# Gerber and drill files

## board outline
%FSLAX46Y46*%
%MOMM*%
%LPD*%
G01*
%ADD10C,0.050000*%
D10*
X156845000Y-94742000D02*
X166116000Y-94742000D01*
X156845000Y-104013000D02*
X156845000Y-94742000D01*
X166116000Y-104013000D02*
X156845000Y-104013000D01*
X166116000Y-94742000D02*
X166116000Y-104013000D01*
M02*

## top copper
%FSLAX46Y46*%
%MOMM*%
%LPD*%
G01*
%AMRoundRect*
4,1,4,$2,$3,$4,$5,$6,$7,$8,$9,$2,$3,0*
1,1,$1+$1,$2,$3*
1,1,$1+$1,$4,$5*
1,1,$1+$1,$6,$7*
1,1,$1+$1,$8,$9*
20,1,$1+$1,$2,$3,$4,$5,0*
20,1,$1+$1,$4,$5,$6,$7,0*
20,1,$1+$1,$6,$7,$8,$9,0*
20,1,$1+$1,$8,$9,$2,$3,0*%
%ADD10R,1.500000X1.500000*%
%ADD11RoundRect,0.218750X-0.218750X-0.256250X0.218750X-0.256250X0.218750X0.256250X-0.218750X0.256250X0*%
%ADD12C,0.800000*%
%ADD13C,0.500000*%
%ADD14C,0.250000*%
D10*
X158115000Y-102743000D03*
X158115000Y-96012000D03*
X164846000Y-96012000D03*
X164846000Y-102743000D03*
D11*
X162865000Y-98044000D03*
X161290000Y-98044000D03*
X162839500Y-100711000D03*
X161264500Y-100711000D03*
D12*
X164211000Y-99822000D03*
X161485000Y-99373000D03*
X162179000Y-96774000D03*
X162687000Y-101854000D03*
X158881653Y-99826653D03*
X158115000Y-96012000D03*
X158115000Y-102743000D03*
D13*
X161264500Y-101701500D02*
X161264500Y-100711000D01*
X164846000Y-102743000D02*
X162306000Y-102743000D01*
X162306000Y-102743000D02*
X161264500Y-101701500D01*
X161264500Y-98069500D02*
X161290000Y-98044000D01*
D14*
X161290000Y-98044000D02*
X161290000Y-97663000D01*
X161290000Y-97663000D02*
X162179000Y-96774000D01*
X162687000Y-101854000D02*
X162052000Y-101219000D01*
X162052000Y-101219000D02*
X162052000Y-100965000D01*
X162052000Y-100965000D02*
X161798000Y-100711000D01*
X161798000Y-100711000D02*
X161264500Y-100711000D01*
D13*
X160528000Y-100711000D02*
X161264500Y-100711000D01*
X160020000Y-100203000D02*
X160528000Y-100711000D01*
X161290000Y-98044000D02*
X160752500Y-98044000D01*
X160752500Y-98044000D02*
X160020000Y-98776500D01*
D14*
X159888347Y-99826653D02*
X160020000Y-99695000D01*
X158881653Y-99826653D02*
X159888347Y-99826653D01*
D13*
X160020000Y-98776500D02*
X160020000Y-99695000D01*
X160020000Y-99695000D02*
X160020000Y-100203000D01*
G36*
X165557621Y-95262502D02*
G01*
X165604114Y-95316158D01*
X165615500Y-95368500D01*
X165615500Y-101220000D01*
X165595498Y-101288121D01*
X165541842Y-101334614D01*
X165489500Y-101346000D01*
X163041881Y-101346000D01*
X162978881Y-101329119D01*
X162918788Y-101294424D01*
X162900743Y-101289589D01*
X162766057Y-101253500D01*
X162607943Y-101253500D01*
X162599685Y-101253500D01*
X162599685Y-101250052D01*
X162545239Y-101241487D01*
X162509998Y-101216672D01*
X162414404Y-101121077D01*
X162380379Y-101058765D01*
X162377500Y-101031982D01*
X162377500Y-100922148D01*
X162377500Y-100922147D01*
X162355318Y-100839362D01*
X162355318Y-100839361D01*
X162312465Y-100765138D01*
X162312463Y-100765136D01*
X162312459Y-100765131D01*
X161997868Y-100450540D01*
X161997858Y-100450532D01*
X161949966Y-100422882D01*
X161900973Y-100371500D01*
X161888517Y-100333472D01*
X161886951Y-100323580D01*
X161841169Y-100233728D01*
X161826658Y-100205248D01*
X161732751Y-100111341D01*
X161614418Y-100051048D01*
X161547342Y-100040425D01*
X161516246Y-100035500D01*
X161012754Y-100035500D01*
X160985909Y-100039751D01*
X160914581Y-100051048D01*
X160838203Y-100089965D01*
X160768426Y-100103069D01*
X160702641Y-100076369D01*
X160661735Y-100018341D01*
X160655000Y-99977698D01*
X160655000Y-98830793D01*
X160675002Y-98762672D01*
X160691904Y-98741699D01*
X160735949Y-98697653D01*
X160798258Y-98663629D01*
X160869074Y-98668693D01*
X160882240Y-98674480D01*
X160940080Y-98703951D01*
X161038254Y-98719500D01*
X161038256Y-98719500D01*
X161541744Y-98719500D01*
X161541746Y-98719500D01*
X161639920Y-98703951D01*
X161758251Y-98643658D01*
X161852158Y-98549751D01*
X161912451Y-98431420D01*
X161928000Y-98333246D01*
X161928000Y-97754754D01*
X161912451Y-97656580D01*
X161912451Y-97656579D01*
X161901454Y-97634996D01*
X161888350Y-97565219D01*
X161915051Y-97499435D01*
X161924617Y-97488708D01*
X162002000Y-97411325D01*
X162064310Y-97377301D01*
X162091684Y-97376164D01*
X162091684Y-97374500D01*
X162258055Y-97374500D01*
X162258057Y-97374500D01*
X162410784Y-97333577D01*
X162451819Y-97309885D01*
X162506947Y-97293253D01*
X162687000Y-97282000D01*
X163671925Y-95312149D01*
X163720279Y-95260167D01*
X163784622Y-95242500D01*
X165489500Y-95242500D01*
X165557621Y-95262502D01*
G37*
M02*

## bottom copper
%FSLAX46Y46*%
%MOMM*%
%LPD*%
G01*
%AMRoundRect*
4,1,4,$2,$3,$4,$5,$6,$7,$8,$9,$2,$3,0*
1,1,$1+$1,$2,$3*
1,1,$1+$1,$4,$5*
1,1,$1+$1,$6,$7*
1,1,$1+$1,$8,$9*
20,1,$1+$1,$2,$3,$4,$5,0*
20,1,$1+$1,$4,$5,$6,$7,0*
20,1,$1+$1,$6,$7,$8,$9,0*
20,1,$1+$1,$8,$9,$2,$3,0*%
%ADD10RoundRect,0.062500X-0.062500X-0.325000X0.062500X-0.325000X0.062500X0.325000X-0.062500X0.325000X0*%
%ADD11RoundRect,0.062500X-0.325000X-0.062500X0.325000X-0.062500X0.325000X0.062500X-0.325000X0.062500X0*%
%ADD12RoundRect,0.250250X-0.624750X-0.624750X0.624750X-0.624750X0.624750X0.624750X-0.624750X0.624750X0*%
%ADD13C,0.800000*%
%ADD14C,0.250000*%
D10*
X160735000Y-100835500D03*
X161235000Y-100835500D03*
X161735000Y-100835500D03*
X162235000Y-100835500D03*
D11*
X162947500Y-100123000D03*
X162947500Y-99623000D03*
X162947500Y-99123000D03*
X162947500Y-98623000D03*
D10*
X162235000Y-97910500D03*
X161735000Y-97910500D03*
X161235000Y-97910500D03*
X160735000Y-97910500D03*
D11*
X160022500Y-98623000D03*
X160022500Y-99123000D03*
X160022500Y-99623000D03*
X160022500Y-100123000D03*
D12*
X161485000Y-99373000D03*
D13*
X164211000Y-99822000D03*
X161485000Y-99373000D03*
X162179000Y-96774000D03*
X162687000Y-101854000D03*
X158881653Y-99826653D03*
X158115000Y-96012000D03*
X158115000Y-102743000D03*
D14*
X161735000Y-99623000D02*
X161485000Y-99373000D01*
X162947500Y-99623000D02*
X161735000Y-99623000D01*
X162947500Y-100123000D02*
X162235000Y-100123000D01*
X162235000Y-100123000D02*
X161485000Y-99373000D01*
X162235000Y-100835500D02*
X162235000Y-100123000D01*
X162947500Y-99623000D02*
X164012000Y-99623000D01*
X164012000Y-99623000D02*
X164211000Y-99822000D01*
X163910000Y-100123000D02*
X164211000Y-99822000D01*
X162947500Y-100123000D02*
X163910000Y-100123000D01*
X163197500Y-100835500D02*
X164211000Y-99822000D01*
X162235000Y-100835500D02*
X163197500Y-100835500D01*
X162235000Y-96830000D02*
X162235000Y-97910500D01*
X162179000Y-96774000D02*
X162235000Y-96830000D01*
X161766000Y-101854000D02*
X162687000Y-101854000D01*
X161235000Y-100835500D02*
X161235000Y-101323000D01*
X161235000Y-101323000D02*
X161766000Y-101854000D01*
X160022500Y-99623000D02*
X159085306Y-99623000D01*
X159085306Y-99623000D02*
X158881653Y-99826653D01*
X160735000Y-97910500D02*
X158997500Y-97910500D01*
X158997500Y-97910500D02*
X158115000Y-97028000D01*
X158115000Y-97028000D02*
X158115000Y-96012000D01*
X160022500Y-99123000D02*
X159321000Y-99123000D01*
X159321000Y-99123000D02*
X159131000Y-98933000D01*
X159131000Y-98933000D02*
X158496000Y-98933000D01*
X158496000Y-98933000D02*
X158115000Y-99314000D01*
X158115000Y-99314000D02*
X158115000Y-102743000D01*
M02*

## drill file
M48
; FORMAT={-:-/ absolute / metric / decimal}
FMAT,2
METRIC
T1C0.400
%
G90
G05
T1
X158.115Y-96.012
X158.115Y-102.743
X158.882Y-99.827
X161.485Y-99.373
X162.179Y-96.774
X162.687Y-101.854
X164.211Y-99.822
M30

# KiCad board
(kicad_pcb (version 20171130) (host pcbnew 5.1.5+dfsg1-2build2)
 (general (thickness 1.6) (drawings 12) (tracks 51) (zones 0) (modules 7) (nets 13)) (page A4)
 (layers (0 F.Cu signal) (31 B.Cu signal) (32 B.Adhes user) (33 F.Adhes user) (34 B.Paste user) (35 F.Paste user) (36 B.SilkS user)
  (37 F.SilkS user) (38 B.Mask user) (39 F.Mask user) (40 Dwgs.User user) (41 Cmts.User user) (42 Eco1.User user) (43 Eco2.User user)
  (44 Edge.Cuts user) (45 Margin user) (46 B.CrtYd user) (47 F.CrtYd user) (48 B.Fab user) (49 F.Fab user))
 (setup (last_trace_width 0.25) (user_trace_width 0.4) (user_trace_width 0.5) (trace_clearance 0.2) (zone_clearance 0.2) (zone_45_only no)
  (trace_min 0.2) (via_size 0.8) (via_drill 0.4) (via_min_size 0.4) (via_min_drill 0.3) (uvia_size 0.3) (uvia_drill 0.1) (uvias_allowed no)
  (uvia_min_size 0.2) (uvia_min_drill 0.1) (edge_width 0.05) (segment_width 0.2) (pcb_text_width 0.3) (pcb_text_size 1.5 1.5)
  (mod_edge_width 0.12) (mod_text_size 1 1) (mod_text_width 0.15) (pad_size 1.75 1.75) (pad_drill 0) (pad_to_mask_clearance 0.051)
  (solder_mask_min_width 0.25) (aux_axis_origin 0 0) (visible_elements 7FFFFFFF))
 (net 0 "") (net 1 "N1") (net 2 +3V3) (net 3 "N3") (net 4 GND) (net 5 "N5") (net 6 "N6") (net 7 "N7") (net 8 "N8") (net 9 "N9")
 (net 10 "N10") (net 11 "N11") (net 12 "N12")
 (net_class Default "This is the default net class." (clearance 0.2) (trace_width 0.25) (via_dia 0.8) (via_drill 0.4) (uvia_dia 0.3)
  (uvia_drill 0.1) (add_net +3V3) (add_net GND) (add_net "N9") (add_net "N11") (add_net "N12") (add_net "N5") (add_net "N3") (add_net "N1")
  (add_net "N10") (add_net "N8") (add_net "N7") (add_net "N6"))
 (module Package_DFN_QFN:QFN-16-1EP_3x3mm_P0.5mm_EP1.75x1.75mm (layer B.Cu) (at 161.485 99.373)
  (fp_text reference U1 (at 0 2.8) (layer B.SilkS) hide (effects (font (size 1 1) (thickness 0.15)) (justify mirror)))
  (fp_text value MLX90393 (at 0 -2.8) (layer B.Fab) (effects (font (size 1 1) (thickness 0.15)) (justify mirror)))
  (pad 16 smd roundrect (at -0.75 1.4625) (size 0.25 0.775) (layers B.Cu B.Paste B.Mask) (roundrect_rratio 0.25) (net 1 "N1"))
  (pad 15 smd roundrect (at -0.25 1.4625) (size 0.25 0.775) (layers B.Cu B.Paste B.Mask) (roundrect_rratio 0.25) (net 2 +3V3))
  (pad 14 smd roundrect (at 0.25 1.4625) (size 0.25 0.775) (layers B.Cu B.Paste B.Mask) (roundrect_rratio 0.25) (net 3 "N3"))
  (pad 13 smd roundrect (at 0.75 1.4625) (size 0.25 0.775) (layers B.Cu B.Paste B.Mask) (roundrect_rratio 0.25) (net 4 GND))
  (pad 12 smd roundrect (at 1.4625 0.75) (size 0.775 0.25) (layers B.Cu B.Paste B.Mask) (roundrect_rratio 0.25) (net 4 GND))
  (pad 11 smd roundrect (at 1.4625 0.25) (size 0.775 0.25) (layers B.Cu B.Paste B.Mask) (roundrect_rratio 0.25) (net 4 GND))
  (pad 10 smd roundrect (at 1.4625 -0.25) (size 0.775 0.25) (layers B.Cu B.Paste B.Mask) (roundrect_rratio 0.25) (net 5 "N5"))
  (pad 9 smd roundrect (at 1.4625 -0.75) (size 0.775 0.25) (layers B.Cu B.Paste B.Mask) (roundrect_rratio 0.25) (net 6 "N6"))
  (pad 8 smd roundrect (at 0.75 -1.4625) (size 0.25 0.775) (layers B.Cu B.Paste B.Mask) (roundrect_rratio 0.25) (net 2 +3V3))
  (pad 7 smd roundrect (at 0.25 -1.4625) (size 0.25 0.775) (layers B.Cu B.Paste B.Mask) (roundrect_rratio 0.25) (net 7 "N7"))
  (pad 6 smd roundrect (at -0.25 -1.4625) (size 0.25 0.775) (layers B.Cu B.Paste B.Mask) (roundrect_rratio 0.25) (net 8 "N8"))
  (pad 5 smd roundrect (at -0.75 -1.4625) (size 0.25 0.775) (layers B.Cu B.Paste B.Mask) (roundrect_rratio 0.25) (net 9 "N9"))
  (pad 4 smd roundrect (at -1.4625 -0.75) (size 0.775 0.25) (layers B.Cu B.Paste B.Mask) (roundrect_rratio 0.25) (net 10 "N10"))
  (pad 3 smd roundrect (at -1.4625 -0.25) (size 0.775 0.25) (layers B.Cu B.Paste B.Mask) (roundrect_rratio 0.25) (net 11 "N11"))
  (pad 2 smd roundrect (at -1.4625 0.25) (size 0.775 0.25) (layers B.Cu B.Paste B.Mask) (roundrect_rratio 0.25) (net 2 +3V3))
  (pad 1 smd roundrect (at -1.4625 0.75) (size 0.775 0.25) (layers B.Cu B.Paste B.Mask) (roundrect_rratio 0.25) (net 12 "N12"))
  (pad "" smd roundrect (at 0.44 -0.44) (size 0.71 0.71) (layers B.Paste) (roundrect_rratio 0.25))
  (pad "" smd roundrect (at 0.44 0.44) (size 0.71 0.71) (layers B.Paste) (roundrect_rratio 0.25))
  (pad "" smd roundrect (at -0.44 -0.44) (size 0.71 0.71) (layers B.Paste) (roundrect_rratio 0.25))
  (pad "" smd roundrect (at -0.44 0.44) (size 0.71 0.71) (layers B.Paste) (roundrect_rratio 0.25))
  (pad 17 smd roundrect (at 0 0) (size 1.75 1.75) (layers B.Cu B.Mask) (roundrect_rratio 0.143) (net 4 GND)))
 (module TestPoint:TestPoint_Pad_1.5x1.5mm (layer F.Cu) (at 158.115 102.743)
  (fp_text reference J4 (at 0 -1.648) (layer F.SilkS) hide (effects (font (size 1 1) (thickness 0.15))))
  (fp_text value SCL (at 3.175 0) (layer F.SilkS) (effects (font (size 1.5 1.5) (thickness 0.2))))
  (pad 1 smd rect (at 0 0) (size 1.5 1.5) (layers F.Cu F.Mask) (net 11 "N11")))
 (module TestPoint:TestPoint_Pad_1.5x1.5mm (layer F.Cu) (at 158.115 96.012)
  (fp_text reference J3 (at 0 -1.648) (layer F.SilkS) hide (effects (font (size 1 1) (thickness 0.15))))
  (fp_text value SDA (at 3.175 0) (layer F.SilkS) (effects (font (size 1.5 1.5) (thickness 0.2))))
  (pad 1 smd rect (at 0 0) (size 1.5 1.5) (layers F.Cu F.Mask) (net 9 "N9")))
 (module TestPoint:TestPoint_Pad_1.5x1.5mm (layer F.Cu) (at 164.846 96.012)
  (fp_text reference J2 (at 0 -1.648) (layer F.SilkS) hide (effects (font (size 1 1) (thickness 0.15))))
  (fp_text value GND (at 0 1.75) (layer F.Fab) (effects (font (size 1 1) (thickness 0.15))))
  (pad 1 smd rect (at 0 0) (size 1.5 1.5) (layers F.Cu F.Mask) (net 4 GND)))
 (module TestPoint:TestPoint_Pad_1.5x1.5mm (layer F.Cu) (at 164.846 102.743)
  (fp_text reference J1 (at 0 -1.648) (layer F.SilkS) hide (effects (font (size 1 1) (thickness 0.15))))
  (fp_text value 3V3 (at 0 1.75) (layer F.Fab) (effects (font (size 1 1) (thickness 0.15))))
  (pad 1 smd rect (at 0 0) (size 1.5 1.5) (layers F.Cu F.Mask) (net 2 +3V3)))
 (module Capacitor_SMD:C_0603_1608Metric (layer F.Cu) (at 162.0775 98.044)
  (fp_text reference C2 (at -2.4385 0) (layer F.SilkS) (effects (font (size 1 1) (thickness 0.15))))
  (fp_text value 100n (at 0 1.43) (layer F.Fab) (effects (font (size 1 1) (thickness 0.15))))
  (pad 2 smd roundrect (at 0.7875 0) (size 0.875 0.95) (layers F.Cu F.Paste F.Mask) (roundrect_rratio 0.25) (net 4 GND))
  (pad 1 smd roundrect (at -0.7875 0) (size 0.875 0.95) (layers F.Cu F.Paste F.Mask) (roundrect_rratio 0.25) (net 2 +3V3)))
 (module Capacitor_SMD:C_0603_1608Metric (layer F.Cu) (at 162.052 100.711)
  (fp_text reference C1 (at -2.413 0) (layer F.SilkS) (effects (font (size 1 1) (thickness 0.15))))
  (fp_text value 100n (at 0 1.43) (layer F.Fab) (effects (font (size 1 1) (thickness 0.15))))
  (pad 2 smd roundrect (at 0.7875 0) (size 0.875 0.95) (layers F.Cu F.Paste F.Mask) (roundrect_rratio 0.25) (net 4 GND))
  (pad 1 smd roundrect (at -0.7875 0) (size 0.875 0.95) (layers F.Cu F.Paste F.Mask) (roundrect_rratio 0.25) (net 2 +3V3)))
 (gr_line (start 156.845 94.742) (end 166.116 94.742) (layer Edge.Cuts) (width 0.05))
 (gr_line (start 156.845 104.013) (end 156.845 94.742) (layer Edge.Cuts) (width 0.05))
 (gr_line (start 166.116 104.013) (end 156.845 104.013) (layer Edge.Cuts) (width 0.05))
 (gr_line (start 166.116 94.742) (end 166.116 104.013) (layer Edge.Cuts) (width 0.05))
 (segment (start 161.735 99.623) (end 161.485 99.373) (width 0.25) (layer B.Cu) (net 4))
 (segment (start 162.9475 99.623) (end 161.735 99.623) (width 0.25) (layer B.Cu) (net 4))
 (segment (start 162.9475 100.123) (end 162.235 100.123) (width 0.25) (layer B.Cu) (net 4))
 (segment (start 162.235 100.123) (end 161.485 99.373) (width 0.25) (layer B.Cu) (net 4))
 (segment (start 162.235 100.8355) (end 162.235 100.123) (width 0.25) (layer B.Cu) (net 4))
 (via (at 164.211 99.822) (size 0.8) (drill 0.4) (layers F.Cu B.Cu) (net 4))
 (segment (start 162.9475 99.623) (end 164.012 99.623) (width 0.25) (layer B.Cu) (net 4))
 (segment (start 164.012 99.623) (end 164.211 99.822) (width 0.25) (layer B.Cu) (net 4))
 (segment (start 163.91 100.123) (end 164.211 99.822) (width 0.25) (layer B.Cu) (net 4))
 (segment (start 162.9475 100.123) (end 163.91 100.123) (width 0.25) (layer B.Cu) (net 4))
 (segment (start 163.1975 100.8355) (end 164.211 99.822) (width 0.25) (layer B.Cu) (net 4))
 (segment (start 162.235 100.8355) (end 163.1975 100.8355) (width 0.25) (layer B.Cu) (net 4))
 (via (at 161.485 99.373) (size 0.8) (drill 0.4) (layers F.Cu B.Cu) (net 4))
 (segment (start 161.2645 101.7015) (end 161.2645 100.711) (width 0.5) (layer F.Cu) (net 2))
 (segment (start 164.846 102.743) (end 162.306 102.743) (width 0.5) (layer F.Cu) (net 2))
 (segment (start 162.306 102.743) (end 161.2645 101.7015) (width 0.5) (layer F.Cu) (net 2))
 (segment (start 161.2645 98.0695) (end 161.29 98.044) (width 0.5) (layer F.Cu) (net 2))
 (via (at 162.179 96.774) (size 0.8) (drill 0.4) (layers F.Cu B.Cu) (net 2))
 (segment (start 161.29 98.044) (end 161.29 97.663) (width 0.25) (layer F.Cu) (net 2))
 (segment (start 161.29 97.663) (end 162.179 96.774) (width 0.25) (layer F.Cu) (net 2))
 (segment (start 162.235 96.83) (end 162.235 97.9105) (width 0.25) (layer B.Cu) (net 2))
 (segment (start 162.179 96.774) (end 162.235 96.83) (width 0.25) (layer B.Cu) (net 2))
 (via (at 162.687 101.854) (size 0.8) (drill 0.4) (layers F.Cu B.Cu) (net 2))
 (segment (start 161.766 101.854) (end 162.687 101.854) (width 0.25) (layer B.Cu) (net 2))
 (segment (start 161.235 100.8355) (end 161.235 101.323) (width 0.25) (layer B.Cu) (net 2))
 (segment (start 161.235 101.323) (end 161.766 101.854) (width 0.25) (layer B.Cu) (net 2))
 (segment (start 162.687 101.854) (end 162.052 101.219) (width 0.25) (layer F.Cu) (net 2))
 (segment (start 162.052 101.219) (end 162.052 100.965) (width 0.25) (layer F.Cu) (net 2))
 (segment (start 162.052 100.965) (end 161.798 100.711) (width 0.25) (layer F.Cu) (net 2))
 (segment (start 161.798 100.711) (end 161.2645 100.711) (width 0.25) (layer F.Cu) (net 2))
 (via (at 158.881653 99.826653) (size 0.8) (drill 0.4) (layers F.Cu B.Cu) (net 2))
 (segment (start 160.0225 99.623) (end 159.085306 99.623) (width 0.25) (layer B.Cu) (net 2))
 (segment (start 159.085306 99.623) (end 158.881653 99.826653) (width 0.25) (layer B.Cu) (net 2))
 (segment (start 160.528 100.711) (end 161.2645 100.711) (width 0.5) (layer F.Cu) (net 2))
 (segment (start 160.02 100.203) (end 160.528 100.711) (width 0.5) (layer F.Cu) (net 2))
 (segment (start 161.29 98.044) (end 160.7525 98.044) (width 0.5) (layer F.Cu) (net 2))
 (segment (start 160.7525 98.044) (end 160.02 98.7765) (width 0.5) (layer F.Cu) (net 2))
 (segment (start 159.888347 99.826653) (end 160.02 99.695) (width 0.25) (layer F.Cu) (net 2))
 (segment (start 158.881653 99.826653) (end 159.888347 99.826653) (width 0.25) (layer F.Cu) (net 2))
 (segment (start 160.02 98.7765) (end 160.02 99.695) (width 0.5) (layer F.Cu) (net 2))
 (segment (start 160.02 99.695) (end 160.02 100.203) (width 0.5) (layer F.Cu) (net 2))
 (segment (start 160.735 97.9105) (end 158.9975 97.9105) (width 0.25) (layer B.Cu) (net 9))
 (via (at 158.115 96.012) (size 0.8) (drill 0.4) (layers F.Cu B.Cu) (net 9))
 (segment (start 158.9975 97.9105) (end 158.115 97.028) (width 0.25) (layer B.Cu) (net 9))
 (segment (start 158.115 97.028) (end 158.115 96.012) (width 0.25) (layer B.Cu) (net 9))
 (segment (start 160.0225 99.123) (end 159.321 99.123) (width 0.25) (layer B.Cu) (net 11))
 (segment (start 159.321 99.123) (end 159.131 98.933) (width 0.25) (layer B.Cu) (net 11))
 (segment (start 159.131 98.933) (end 158.496 98.933) (width 0.25) (layer B.Cu) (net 11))
 (via (at 158.115 102.743) (size 0.8) (drill 0.4) (layers F.Cu B.Cu) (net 11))
 (segment (start 158.496 98.933) (end 158.115 99.314) (width 0.25) (layer B.Cu) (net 11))
 (segment (start 158.115 99.314) (end 158.115 102.743) (width 0.25) (layer B.Cu) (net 11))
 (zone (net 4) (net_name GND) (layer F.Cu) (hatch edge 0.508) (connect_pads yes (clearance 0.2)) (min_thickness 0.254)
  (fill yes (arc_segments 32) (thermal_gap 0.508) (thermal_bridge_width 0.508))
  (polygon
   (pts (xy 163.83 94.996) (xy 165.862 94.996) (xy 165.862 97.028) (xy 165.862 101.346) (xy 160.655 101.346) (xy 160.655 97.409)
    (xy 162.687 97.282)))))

